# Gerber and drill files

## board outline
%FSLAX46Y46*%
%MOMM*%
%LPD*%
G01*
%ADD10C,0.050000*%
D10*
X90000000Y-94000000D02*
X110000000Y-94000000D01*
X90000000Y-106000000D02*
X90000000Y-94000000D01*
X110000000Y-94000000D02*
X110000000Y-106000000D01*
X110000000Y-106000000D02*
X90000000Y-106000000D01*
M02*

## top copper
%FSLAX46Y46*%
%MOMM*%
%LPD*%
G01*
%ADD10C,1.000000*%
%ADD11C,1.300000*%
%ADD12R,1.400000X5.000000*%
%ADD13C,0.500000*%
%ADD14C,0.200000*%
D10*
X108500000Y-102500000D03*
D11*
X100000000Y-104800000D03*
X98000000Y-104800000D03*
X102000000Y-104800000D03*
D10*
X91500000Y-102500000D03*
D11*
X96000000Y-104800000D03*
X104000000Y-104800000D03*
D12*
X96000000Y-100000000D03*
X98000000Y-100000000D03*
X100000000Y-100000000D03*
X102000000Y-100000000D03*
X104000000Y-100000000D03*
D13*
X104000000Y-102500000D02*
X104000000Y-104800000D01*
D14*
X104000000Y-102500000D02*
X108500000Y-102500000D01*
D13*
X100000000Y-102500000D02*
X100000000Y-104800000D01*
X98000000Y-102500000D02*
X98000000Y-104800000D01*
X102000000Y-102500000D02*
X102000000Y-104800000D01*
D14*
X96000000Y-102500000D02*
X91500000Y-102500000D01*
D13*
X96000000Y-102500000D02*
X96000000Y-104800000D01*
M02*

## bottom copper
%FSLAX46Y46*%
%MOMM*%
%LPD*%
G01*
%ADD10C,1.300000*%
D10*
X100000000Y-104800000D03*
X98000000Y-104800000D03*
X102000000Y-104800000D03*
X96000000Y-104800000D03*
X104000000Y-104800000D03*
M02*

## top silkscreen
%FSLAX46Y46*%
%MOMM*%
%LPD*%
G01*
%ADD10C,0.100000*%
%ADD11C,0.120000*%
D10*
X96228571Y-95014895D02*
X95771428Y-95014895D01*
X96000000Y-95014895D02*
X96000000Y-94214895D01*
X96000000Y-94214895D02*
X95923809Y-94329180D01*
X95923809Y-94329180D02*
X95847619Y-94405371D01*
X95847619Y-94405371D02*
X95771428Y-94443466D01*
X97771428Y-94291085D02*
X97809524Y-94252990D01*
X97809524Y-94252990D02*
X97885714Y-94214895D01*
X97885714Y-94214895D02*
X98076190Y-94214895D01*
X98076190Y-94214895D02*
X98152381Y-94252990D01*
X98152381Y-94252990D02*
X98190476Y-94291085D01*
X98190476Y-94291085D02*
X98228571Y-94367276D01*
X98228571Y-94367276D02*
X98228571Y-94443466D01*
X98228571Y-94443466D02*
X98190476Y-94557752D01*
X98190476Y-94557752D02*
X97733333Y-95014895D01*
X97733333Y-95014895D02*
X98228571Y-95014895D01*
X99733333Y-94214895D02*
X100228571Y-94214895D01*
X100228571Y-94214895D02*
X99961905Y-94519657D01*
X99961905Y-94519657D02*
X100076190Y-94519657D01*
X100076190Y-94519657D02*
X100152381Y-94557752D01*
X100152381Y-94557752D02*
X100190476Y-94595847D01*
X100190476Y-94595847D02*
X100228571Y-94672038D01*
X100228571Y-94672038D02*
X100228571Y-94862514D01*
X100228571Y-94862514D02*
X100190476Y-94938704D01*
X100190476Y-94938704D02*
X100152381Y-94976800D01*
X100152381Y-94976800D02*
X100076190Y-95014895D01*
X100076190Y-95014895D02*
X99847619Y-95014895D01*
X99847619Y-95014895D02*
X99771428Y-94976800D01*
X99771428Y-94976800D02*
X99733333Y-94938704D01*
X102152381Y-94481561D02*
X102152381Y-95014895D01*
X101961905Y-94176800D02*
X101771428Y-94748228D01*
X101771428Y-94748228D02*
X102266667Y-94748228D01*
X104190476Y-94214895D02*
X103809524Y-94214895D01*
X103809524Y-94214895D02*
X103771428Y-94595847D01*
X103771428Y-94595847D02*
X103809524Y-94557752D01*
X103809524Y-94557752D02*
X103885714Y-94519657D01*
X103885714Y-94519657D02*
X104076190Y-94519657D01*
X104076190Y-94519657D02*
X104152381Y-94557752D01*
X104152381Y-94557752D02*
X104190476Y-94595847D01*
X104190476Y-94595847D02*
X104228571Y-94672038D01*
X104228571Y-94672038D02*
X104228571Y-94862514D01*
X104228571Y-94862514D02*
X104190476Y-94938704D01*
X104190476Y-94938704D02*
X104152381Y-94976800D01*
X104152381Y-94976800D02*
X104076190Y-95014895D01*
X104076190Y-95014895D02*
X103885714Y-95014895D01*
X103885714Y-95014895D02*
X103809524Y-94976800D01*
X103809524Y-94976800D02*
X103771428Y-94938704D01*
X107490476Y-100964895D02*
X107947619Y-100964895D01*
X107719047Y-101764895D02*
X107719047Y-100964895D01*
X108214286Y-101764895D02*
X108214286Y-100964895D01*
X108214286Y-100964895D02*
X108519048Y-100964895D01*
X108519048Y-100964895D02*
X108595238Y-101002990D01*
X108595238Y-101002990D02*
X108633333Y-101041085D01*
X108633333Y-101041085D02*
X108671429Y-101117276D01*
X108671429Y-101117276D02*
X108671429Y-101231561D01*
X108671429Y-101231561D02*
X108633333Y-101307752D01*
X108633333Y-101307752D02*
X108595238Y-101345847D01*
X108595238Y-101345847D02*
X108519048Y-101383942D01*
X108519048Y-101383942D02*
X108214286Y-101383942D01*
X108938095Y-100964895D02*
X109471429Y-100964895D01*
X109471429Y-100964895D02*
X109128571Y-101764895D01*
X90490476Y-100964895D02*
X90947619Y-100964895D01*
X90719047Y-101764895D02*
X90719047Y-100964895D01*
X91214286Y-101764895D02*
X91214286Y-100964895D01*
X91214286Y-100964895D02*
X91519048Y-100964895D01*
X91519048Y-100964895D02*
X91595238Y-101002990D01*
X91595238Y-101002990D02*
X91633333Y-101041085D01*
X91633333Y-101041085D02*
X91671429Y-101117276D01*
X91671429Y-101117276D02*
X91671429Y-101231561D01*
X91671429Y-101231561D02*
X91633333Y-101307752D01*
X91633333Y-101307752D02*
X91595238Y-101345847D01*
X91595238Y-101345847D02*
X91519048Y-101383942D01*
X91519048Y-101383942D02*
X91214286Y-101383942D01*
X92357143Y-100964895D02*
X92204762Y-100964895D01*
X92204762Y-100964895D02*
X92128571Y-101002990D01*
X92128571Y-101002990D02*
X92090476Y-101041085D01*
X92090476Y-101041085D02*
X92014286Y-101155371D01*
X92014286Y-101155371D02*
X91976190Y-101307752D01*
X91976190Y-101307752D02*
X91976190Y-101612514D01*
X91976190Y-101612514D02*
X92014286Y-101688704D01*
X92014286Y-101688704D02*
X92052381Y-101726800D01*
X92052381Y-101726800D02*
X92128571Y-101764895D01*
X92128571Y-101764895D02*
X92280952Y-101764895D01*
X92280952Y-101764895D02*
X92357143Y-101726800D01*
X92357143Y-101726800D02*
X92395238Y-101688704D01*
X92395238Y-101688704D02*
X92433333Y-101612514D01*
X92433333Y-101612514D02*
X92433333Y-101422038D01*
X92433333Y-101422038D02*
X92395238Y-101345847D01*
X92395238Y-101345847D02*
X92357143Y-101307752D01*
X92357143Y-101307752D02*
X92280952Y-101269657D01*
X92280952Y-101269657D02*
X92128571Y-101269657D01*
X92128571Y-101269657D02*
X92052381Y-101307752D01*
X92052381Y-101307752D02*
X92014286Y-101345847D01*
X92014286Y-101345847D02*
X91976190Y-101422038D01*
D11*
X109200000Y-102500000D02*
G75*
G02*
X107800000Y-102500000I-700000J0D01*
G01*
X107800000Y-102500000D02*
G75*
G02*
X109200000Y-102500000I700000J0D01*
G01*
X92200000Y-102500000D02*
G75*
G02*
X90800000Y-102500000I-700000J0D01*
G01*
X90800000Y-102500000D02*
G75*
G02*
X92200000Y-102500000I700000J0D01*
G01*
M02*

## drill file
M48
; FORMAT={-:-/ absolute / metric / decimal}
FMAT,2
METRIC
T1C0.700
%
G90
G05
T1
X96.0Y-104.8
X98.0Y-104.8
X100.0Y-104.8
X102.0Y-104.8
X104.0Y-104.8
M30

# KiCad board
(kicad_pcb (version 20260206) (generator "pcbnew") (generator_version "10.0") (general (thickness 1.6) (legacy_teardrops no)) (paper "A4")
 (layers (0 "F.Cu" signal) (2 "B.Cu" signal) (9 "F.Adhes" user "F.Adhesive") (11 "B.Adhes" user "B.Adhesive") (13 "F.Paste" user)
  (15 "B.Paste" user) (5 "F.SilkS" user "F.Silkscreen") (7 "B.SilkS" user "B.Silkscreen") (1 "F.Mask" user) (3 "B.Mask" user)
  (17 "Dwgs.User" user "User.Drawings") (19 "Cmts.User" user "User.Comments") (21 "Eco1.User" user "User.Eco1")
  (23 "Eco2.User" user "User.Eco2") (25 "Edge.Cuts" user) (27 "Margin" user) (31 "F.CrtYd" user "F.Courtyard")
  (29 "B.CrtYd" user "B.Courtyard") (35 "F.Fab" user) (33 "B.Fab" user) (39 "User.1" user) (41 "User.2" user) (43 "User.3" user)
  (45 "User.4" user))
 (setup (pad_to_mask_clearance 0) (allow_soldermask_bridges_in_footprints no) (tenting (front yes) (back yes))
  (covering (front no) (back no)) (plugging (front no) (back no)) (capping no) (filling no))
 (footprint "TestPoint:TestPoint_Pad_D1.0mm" (layer "F.Cu") (at 108.5 102.5)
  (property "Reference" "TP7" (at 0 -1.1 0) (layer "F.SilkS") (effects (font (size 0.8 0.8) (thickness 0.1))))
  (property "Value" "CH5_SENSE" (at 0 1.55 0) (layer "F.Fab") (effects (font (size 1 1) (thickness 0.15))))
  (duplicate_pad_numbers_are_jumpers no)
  (fp_circle (center 0 0) (end 0 0.7) (stroke (width 0.12) (type solid)) (fill no) (layer "F.SilkS"))
  (pad "1" smd circle (at 0 0) (size 1 1) (layers "F.Cu" "F.Mask") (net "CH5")))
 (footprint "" (layer "F.Cu") (at 100 104.8)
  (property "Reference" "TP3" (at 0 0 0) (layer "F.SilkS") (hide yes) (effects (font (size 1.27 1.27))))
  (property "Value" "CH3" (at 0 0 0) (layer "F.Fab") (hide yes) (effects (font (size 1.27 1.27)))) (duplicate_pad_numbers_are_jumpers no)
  (pad "1" thru_hole circle (at 0 0) (size 1.3 1.3) (drill 0.7) (layers "*.Cu") (remove_unused_layers no) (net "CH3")))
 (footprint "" (layer "F.Cu") (at 98 104.8)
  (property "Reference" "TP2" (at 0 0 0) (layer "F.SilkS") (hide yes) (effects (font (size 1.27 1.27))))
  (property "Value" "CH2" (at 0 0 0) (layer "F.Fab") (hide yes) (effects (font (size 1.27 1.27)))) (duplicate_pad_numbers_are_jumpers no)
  (pad "1" thru_hole circle (at 0 0) (size 1.3 1.3) (drill 0.7) (layers "*.Cu") (remove_unused_layers no) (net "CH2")))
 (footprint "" (layer "F.Cu") (at 102 104.8)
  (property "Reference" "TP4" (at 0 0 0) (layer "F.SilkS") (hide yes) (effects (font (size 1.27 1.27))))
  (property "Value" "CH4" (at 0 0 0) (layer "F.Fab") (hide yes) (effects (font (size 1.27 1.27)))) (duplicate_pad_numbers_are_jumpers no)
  (pad "1" thru_hole circle (at 0 0) (size 1.3 1.3) (drill 0.7) (layers "*.Cu") (remove_unused_layers no) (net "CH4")))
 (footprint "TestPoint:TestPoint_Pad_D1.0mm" (layer "F.Cu") (at 91.5 102.5)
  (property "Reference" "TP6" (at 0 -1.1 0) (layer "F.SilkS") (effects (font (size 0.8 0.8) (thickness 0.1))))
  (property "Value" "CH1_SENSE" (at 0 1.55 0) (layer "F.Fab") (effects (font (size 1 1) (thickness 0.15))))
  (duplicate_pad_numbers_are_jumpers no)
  (fp_circle (center 0 0) (end 0 0.7) (stroke (width 0.12) (type solid)) (fill no) (layer "F.SilkS"))
  (pad "1" smd circle (at 0 0) (size 1 1) (layers "F.Cu" "F.Mask") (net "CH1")))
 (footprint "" (layer "F.Cu") (at 96 104.8)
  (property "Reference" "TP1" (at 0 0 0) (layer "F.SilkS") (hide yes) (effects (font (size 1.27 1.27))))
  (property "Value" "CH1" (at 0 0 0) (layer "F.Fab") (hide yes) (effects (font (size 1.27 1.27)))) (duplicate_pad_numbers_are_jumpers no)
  (pad "1" thru_hole circle (at 0 0) (size 1.3 1.3) (drill 0.7) (layers "*.Cu") (remove_unused_layers no) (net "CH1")))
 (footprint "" (layer "F.Cu") (at 104 104.8)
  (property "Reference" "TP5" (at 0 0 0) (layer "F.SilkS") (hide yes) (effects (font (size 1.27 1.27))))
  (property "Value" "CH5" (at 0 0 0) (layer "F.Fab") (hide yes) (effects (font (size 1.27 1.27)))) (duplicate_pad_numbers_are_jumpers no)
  (pad "1" thru_hole circle (at 0 0) (size 1.3 1.3) (drill 0.7) (layers "*.Cu") (remove_unused_layers no) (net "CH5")))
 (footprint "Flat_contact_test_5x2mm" (layer "F.Cu") (at 100 100)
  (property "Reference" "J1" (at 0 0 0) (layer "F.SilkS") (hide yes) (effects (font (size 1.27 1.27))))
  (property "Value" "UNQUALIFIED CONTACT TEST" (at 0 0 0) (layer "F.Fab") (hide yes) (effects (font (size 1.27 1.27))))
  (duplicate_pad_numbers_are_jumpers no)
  (pad "1" smd rect (at -4 0) (size 1.4 5) (layers "F.Cu" "F.Mask") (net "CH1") (thermal_bridge_angle 45))
  (pad "2" smd rect (at -2 0) (size 1.4 5) (layers "F.Cu" "F.Mask") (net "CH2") (thermal_bridge_angle 45))
  (pad "3" smd rect (at 0 0) (size 1.4 5) (layers "F.Cu" "F.Mask") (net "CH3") (thermal_bridge_angle 45))
  (pad "4" smd rect (at 2 0) (size 1.4 5) (layers "F.Cu" "F.Mask") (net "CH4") (thermal_bridge_angle 45))
  (pad "5" smd rect (at 4 0) (size 1.4 5) (layers "F.Cu" "F.Mask") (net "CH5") (thermal_bridge_angle 45)))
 (gr_line (start 90 94) (end 110 94) (stroke (width 0.05) (type default)) (layer "Edge.Cuts"))
 (gr_line (start 90 106) (end 90 94) (stroke (width 0.05) (type default)) (layer "Edge.Cuts"))
 (gr_line (start 110 94) (end 110 106) (stroke (width 0.05) (type default)) (layer "Edge.Cuts"))
 (gr_line (start 110 106) (end 90 106) (stroke (width 0.05) (type default)) (layer "Edge.Cuts"))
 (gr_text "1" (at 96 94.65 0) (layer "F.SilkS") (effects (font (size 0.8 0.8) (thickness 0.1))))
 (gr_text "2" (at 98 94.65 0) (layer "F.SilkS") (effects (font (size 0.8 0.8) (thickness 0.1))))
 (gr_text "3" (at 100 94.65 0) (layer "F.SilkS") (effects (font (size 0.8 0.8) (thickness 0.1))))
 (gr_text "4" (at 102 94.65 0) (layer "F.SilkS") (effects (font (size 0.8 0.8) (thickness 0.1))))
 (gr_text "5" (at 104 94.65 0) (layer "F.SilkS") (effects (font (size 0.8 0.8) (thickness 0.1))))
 (segment (start 104 102.5) (end 104 104.8) (width 0.5) (layer "F.Cu") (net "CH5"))
 (segment (start 104 102.5) (end 108.5 102.5) (width 0.2) (layer "F.Cu") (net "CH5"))
 (segment (start 100 102.5) (end 100 104.8) (width 0.5) (layer "F.Cu") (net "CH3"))
 (segment (start 98 102.5) (end 98 104.8) (width 0.5) (layer "F.Cu") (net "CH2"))
 (segment (start 102 102.5) (end 102 104.8) (width 0.5) (layer "F.Cu") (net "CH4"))
 (segment (start 96 102.5) (end 91.5 102.5) (width 0.2) (layer "F.Cu") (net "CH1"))
 (segment (start 96 102.5) (end 96 104.8) (width 0.5) (layer "F.Cu") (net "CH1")))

